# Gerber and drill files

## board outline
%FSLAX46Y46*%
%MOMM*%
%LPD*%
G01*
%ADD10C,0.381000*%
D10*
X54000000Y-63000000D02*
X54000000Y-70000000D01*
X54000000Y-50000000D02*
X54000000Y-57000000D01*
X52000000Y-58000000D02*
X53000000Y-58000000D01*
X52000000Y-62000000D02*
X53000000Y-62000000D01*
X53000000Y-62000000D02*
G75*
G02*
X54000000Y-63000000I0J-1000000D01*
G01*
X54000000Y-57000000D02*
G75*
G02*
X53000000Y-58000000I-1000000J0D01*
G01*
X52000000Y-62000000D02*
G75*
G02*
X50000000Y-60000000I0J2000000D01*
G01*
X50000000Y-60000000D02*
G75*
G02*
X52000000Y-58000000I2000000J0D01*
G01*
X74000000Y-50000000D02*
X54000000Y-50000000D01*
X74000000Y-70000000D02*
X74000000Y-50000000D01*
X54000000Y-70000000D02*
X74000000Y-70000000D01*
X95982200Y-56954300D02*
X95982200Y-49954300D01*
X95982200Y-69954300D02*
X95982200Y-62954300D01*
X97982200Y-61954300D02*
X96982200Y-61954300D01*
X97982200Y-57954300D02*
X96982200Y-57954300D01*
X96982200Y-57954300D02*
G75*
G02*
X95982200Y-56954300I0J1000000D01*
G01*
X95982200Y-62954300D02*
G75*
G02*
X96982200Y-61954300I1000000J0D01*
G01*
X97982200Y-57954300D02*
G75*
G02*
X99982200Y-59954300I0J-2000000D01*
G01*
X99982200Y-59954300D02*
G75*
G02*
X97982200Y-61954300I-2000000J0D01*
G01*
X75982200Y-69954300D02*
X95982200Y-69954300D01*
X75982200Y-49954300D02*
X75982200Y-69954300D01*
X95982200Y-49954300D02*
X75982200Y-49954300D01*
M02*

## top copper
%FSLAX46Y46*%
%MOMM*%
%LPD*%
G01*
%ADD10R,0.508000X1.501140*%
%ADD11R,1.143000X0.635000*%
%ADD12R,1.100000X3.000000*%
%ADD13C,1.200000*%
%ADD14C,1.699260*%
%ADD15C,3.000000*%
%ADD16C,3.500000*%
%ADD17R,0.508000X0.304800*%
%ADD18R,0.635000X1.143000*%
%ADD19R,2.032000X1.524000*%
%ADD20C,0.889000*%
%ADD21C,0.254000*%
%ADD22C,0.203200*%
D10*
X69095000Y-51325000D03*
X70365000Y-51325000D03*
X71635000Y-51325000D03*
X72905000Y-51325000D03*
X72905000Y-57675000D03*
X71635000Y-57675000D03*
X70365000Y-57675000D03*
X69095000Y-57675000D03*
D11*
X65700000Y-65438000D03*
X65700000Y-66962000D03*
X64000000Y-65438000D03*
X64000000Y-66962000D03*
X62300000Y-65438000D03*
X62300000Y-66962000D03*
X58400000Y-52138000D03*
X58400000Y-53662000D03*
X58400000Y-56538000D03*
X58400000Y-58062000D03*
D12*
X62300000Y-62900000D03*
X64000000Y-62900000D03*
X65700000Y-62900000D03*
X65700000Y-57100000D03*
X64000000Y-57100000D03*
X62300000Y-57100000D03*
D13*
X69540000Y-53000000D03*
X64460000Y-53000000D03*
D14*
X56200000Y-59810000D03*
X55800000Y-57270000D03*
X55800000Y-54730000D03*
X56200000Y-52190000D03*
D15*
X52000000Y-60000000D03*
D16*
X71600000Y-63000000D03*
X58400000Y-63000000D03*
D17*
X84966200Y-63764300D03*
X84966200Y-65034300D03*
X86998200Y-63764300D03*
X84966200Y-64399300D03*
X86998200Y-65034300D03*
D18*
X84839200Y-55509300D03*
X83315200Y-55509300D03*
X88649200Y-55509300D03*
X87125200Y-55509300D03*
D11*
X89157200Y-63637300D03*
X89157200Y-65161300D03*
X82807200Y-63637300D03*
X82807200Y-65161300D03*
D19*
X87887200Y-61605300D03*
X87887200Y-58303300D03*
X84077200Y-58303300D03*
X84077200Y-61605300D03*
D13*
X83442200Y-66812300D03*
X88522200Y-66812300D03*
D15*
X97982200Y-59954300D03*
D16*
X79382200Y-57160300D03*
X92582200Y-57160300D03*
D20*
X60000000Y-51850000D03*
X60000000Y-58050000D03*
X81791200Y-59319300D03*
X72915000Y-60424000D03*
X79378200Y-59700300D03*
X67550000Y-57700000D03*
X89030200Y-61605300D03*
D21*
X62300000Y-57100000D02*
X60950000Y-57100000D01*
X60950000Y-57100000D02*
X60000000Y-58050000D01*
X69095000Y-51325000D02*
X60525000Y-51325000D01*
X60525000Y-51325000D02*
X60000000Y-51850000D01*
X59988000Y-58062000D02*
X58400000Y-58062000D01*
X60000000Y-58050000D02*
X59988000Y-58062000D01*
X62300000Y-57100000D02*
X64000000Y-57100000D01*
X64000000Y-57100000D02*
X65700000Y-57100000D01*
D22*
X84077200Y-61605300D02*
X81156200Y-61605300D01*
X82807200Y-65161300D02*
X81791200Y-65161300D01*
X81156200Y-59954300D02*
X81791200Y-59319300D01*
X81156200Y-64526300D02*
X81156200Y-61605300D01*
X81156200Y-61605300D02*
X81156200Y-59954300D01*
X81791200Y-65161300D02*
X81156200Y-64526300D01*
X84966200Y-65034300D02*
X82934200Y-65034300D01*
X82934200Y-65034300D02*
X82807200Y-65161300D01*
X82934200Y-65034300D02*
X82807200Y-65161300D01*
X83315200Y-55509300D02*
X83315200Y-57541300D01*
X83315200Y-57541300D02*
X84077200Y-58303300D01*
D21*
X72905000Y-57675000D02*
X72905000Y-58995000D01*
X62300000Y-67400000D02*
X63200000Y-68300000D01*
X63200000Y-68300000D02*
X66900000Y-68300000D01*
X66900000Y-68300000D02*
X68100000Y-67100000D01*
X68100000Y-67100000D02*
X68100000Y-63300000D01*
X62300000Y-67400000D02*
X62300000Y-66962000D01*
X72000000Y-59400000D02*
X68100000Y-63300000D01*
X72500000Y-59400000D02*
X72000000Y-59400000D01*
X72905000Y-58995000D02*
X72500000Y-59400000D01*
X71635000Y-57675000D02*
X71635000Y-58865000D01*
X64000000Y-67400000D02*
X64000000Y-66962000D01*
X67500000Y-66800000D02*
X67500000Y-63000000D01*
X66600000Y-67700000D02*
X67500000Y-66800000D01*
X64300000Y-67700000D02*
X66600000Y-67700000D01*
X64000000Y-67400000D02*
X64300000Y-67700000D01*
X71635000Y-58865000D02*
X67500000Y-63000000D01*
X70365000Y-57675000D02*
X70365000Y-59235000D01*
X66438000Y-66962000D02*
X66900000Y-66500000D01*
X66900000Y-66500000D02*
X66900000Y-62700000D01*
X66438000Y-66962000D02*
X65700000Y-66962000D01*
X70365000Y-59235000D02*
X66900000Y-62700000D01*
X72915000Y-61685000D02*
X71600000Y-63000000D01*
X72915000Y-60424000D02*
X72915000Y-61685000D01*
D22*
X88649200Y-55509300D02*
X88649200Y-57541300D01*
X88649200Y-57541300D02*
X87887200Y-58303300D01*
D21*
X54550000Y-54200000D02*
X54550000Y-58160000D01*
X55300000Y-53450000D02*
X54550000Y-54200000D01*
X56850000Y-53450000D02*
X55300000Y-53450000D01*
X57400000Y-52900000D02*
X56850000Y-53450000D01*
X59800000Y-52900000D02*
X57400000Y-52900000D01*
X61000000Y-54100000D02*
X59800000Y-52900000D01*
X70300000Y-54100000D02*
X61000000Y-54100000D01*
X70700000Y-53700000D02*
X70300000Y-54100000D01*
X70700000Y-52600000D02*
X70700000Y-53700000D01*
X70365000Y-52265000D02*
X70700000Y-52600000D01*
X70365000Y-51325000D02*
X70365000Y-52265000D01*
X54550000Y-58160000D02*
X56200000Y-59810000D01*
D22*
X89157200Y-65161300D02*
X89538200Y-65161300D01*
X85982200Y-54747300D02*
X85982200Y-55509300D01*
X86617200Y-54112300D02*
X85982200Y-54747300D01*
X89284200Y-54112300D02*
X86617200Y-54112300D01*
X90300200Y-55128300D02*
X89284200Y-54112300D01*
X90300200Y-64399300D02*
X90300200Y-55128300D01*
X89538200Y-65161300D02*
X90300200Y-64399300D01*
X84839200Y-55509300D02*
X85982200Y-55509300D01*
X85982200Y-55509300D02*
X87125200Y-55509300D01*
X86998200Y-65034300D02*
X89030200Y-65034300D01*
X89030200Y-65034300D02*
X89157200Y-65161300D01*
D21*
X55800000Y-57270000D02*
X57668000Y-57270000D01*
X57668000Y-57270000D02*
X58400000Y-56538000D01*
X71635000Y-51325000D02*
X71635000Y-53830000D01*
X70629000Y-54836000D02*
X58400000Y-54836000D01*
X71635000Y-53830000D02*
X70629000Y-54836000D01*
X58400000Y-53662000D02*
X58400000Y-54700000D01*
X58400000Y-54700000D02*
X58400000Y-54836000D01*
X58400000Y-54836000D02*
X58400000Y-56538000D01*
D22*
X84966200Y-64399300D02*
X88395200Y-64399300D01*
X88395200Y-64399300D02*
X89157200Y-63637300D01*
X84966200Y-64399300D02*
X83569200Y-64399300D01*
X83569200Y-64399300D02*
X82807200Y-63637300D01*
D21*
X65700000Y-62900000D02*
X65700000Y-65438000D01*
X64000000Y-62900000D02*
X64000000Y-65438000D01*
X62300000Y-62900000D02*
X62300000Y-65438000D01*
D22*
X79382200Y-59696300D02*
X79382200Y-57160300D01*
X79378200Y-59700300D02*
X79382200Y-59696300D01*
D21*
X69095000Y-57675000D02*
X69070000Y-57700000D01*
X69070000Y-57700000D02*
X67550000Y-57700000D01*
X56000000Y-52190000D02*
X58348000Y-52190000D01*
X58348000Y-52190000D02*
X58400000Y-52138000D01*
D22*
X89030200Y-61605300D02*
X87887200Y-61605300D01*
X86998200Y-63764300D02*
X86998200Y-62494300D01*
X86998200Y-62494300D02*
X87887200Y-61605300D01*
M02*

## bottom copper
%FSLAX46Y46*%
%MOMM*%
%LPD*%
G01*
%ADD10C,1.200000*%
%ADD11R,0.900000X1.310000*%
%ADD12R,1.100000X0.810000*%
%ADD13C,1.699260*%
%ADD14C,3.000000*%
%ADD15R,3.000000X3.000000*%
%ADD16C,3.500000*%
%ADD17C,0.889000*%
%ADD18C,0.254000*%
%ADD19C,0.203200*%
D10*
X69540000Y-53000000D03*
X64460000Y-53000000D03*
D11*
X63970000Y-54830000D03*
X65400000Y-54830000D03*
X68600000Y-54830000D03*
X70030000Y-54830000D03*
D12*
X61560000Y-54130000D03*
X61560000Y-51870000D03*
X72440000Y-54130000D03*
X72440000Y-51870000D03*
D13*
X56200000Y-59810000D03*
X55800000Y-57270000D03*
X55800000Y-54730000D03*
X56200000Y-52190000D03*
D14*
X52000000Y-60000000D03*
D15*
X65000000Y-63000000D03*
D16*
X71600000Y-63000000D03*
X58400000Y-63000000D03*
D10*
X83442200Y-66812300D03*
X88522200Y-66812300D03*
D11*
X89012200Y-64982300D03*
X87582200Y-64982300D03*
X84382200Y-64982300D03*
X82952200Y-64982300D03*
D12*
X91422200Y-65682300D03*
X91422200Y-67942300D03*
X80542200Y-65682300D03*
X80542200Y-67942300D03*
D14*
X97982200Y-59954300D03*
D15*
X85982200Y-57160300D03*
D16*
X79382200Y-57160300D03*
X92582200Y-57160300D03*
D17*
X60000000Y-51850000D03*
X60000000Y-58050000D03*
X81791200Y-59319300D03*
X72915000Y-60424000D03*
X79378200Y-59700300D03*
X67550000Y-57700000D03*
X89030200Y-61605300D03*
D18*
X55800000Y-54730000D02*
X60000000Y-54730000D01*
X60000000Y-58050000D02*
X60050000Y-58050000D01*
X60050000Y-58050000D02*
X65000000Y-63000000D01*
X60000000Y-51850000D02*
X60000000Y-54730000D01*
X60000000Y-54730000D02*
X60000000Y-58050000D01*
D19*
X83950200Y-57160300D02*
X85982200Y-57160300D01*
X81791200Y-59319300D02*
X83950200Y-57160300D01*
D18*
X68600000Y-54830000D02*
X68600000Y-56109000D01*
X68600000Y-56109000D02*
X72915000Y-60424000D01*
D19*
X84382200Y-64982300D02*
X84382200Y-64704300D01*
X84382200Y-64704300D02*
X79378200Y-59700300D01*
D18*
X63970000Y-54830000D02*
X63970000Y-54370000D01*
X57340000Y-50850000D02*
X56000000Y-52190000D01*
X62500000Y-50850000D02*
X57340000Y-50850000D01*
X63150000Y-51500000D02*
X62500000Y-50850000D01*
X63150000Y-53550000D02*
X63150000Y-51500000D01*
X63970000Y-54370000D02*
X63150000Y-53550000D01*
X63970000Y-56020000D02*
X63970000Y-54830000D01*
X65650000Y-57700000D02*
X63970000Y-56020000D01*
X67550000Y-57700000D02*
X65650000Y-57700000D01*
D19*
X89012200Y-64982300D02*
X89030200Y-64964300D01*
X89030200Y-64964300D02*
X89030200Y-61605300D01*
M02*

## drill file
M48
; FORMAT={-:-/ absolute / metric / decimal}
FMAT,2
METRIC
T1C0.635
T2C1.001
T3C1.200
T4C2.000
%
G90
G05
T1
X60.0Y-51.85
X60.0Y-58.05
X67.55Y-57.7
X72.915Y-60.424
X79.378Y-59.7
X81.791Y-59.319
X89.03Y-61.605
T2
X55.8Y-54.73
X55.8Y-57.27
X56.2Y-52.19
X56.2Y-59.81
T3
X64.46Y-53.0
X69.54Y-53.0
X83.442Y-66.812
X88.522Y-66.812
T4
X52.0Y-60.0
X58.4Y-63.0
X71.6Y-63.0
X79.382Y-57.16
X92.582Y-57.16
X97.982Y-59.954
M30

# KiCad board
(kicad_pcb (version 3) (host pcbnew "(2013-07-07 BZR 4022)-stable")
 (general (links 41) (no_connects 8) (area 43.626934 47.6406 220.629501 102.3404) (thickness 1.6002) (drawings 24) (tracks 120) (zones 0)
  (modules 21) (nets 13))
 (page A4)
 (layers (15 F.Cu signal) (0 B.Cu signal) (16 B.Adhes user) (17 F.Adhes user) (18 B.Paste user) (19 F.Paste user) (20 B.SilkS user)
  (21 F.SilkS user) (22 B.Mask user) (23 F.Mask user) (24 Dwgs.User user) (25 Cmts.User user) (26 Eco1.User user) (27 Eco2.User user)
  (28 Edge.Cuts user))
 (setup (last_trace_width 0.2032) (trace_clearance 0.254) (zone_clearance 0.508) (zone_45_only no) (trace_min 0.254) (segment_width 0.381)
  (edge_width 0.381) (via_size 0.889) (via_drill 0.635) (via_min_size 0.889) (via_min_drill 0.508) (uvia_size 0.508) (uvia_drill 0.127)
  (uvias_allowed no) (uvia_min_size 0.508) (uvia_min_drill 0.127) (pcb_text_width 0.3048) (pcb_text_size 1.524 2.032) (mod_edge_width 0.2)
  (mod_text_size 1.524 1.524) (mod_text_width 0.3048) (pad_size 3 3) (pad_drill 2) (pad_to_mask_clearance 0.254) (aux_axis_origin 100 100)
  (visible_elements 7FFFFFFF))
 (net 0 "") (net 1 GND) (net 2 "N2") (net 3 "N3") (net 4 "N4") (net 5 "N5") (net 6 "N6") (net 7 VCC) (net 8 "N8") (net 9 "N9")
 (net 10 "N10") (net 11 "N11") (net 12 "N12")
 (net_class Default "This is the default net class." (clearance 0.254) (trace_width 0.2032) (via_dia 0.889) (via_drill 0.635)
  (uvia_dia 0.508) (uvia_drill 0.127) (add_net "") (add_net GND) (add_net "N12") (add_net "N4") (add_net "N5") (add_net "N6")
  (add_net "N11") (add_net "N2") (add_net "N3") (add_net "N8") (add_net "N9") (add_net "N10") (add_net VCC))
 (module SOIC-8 (layer F.Cu) (at 71 54.5)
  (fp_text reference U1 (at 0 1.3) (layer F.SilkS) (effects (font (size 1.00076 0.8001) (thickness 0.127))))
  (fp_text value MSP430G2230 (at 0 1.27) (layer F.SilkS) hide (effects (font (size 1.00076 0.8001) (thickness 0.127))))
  (pad 8 smd rect (at -1.905 -3.175) (size 0.508 1.50114) (layers F.Cu F.Paste F.Mask) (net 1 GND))
  (pad 7 smd rect (at -0.635 -3.175) (size 0.508 1.50114) (layers F.Cu F.Paste F.Mask) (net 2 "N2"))
  (pad 6 smd rect (at 0.635 -3.175) (size 0.508 1.50114) (layers F.Cu F.Paste F.Mask) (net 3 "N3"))
  (pad 5 smd rect (at 1.905 -3.175) (size 0.508 1.50114) (layers F.Cu F.Paste F.Mask))
  (pad 4 smd rect (at 1.905 3.175) (size 0.508 1.50114) (layers F.Cu F.Paste F.Mask) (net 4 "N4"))
  (pad 3 smd rect (at 0.635 3.175) (size 0.508 1.50114) (layers F.Cu F.Paste F.Mask) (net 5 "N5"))
  (pad 2 smd rect (at -0.635 3.175) (size 0.508 1.50114) (layers F.Cu F.Paste F.Mask) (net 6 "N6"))
  (pad 1 smd rect (at -1.905 3.175) (size 0.508 1.50114) (layers F.Cu F.Paste F.Mask) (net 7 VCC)))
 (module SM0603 (layer F.Cu) (at 65.7 66.2 270)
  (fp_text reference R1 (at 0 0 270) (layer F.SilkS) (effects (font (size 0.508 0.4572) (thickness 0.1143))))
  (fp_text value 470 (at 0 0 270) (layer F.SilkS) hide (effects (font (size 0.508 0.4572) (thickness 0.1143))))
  (pad 1 smd rect (at -0.762 0 270) (size 0.635 1.143) (layers F.Cu F.Paste F.Mask) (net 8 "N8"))
  (pad 2 smd rect (at 0.762 0 270) (size 0.635 1.143) (layers F.Cu F.Paste F.Mask) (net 6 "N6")))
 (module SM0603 (layer F.Cu) (at 64 66.2 270)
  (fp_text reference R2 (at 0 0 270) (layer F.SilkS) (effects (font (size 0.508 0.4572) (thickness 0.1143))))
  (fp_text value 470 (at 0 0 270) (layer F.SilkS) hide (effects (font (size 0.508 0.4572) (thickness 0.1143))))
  (pad 1 smd rect (at -0.762 0 270) (size 0.635 1.143) (layers F.Cu F.Paste F.Mask) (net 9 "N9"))
  (pad 2 smd rect (at 0.762 0 270) (size 0.635 1.143) (layers F.Cu F.Paste F.Mask) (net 5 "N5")))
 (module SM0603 (layer F.Cu) (at 62.3 66.2 270)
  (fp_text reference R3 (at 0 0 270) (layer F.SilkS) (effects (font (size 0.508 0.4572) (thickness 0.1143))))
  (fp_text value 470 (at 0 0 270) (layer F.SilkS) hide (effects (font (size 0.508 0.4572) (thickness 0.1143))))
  (pad 1 smd rect (at -0.762 0 270) (size 0.635 1.143) (layers F.Cu F.Paste F.Mask) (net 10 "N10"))
  (pad 2 smd rect (at 0.762 0 270) (size 0.635 1.143) (layers F.Cu F.Paste F.Mask) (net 4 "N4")))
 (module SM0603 (layer F.Cu) (at 58.4 52.9 270)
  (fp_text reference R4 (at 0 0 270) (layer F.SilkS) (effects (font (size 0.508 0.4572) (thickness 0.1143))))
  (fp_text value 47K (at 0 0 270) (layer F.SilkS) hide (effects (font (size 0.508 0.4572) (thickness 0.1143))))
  (pad 1 smd rect (at -0.762 0 270) (size 0.635 1.143) (layers F.Cu F.Paste F.Mask) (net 7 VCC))
  (pad 2 smd rect (at 0.762 0 270) (size 0.635 1.143) (layers F.Cu F.Paste F.Mask) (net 3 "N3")))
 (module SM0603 (layer F.Cu) (at 58.4 57.3 270)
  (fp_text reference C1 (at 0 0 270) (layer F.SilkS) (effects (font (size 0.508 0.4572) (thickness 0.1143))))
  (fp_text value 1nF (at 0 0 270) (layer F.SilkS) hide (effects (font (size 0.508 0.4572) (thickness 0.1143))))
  (pad 1 smd rect (at -0.762 0 270) (size 0.635 1.143) (layers F.Cu F.Paste F.Mask) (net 3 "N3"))
  (pad 2 smd rect (at 0.762 0 270) (size 0.635 1.143) (layers F.Cu F.Paste F.Mask) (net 1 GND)))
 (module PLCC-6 (layer F.Cu) (at 64 60)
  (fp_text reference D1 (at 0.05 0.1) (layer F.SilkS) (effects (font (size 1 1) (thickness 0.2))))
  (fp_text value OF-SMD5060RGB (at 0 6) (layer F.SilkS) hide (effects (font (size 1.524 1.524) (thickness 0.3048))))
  (pad 1 smd rect (at -1.7 2.9) (size 1.1 3) (layers F.Cu F.Paste F.Mask) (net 10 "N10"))
  (pad 2 smd rect (at 0 2.9) (size 1.1 3) (layers F.Cu F.Paste F.Mask) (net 9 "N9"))
  (pad 3 smd rect (at 1.7 2.9) (size 1.1 3) (layers F.Cu F.Paste F.Mask) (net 8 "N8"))
  (pad 4 smd rect (at 1.7 -2.9) (size 1.1 3) (layers F.Cu F.Paste F.Mask) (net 1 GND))
  (pad 5 smd rect (at 0 -2.9) (size 1.1 3) (layers F.Cu F.Paste F.Mask) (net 1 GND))
  (pad 6 smd rect (at -1.7 -2.9) (size 1.1 3) (layers F.Cu F.Paste F.Mask) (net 1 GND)))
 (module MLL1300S (layer B.Cu) (at 67 53)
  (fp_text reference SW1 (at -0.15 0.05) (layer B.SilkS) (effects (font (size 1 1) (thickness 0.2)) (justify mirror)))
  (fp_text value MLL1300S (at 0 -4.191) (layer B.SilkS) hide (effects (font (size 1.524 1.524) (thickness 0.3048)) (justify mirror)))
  (pad ~ thru_hole circle (at 2.54 0) (size 1.2 1.2) (drill 1.2) (layers *.Cu *.Mask B.SilkS))
  (pad ~ thru_hole circle (at -2.54 0) (size 1.2 1.2) (drill 1.2) (layers *.Cu *.Mask B.SilkS))
  (pad 1 smd rect (at -3.03 1.83) (size 0.9 1.31) (layers B.Cu B.Paste B.Mask) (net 7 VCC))
  (pad 2 smd rect (at -1.6 1.83) (size 0.9 1.31) (layers B.Cu B.Paste B.Mask))
  (pad 3 smd rect (at 1.6 1.83) (size 0.9 1.31) (layers B.Cu B.Paste B.Mask) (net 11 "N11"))
  (pad 4 smd rect (at 3.03 1.83) (size 0.9 1.31) (layers B.Cu B.Paste B.Mask))
  (pad ~ smd rect (at -5.44 1.13) (size 1.1 0.81) (layers B.Cu B.Paste B.Mask))
  (pad ~ smd rect (at -5.44 -1.13) (size 1.1 0.81) (layers B.Cu B.Paste B.Mask))
  (pad ~ smd rect (at 5.44 1.13) (size 1.1 0.81) (layers B.Cu B.Paste B.Mask))
  (pad ~ smd rect (at 5.44 -1.13) (size 1.1 0.81) (layers B.Cu B.Paste B.Mask)))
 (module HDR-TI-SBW (layer F.Cu) (at 56 56 90)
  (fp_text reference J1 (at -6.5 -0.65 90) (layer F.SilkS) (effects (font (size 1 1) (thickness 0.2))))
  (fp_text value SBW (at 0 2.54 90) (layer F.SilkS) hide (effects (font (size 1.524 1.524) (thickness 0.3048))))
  (pad 1 thru_hole circle (at -3.81 0.2 90) (size 1.69926 1.69926) (drill 1.00076) (layers *.Cu *.Mask F.SilkS) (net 2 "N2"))
  (pad 2 thru_hole circle (at -1.27 -0.2 90) (size 1.69926 1.69926) (drill 1.00076) (layers *.Cu *.Mask F.SilkS) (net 3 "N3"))
  (pad 3 thru_hole circle (at 1.27 -0.2 90) (size 1.69926 1.69926) (drill 1.00076) (layers *.Cu *.Mask F.SilkS) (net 1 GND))
  (pad 4 thru_hole circle (at 3.81 0.2 90) (size 1.69926 1.69926) (drill 1.00076) (layers *.Cu *.Mask F.SilkS) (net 7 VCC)))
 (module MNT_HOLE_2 (layer F.Cu) (at 52 60)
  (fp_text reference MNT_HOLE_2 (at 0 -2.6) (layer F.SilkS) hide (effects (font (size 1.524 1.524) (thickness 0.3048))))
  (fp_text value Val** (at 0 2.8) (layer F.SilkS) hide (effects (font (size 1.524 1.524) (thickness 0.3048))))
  (pad "" thru_hole circle (at 0 0) (size 3 3) (drill 2) (layers *.Cu *.Mask F.SilkS)))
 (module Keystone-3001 (layer B.Cu) (at 65 63)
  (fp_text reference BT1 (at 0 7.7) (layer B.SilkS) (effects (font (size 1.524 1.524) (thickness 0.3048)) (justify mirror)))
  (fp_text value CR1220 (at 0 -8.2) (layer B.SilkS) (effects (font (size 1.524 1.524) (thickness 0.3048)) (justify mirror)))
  (pad 2 smd rect (at 0 0) (size 3 3) (layers B.Cu B.Paste B.Mask) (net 1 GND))
  (pad 1 thru_hole circle (at 6.6 0) (size 3.5 3.5) (drill 2) (layers F.Cu F.Mask) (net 11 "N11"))
  (pad 1 thru_hole circle (at -6.6 0) (size 3.5 3.5) (drill 2) (layers F.Cu F.Mask) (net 11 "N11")))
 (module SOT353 (layer F.Cu) (at 85.9822 64.3993)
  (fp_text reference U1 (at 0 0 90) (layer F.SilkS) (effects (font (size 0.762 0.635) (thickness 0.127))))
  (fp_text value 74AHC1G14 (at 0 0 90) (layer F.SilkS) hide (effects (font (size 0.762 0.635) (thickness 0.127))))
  (pad 1 smd rect (at -1.016 -0.635) (size 0.508 0.3048) (layers F.Cu F.Paste F.Mask))
  (pad 3 smd rect (at -1.016 0.635) (size 0.508 0.3048) (layers F.Cu F.Paste F.Mask) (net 1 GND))
  (pad 5 smd rect (at 1.016 -0.635) (size 0.508 0.3048) (layers F.Cu F.Paste F.Mask) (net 7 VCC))
  (pad 2 smd rect (at -1.016 0) (size 0.508 0.3048) (layers F.Cu F.Paste F.Mask) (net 3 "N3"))
  (pad 4 smd rect (at 1.016 0.635) (size 0.508 0.3048) (layers F.Cu F.Paste F.Mask) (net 2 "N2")))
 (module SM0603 (layer F.Cu) (at 84.0772 55.5093 180)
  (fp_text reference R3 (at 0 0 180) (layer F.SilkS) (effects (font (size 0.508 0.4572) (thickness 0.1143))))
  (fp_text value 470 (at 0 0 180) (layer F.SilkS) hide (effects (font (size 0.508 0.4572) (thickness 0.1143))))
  (pad 1 smd rect (at -0.762 0 180) (size 0.635 1.143) (layers F.Cu F.Paste F.Mask) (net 2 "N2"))
  (pad 2 smd rect (at 0.762 0 180) (size 0.635 1.143) (layers F.Cu F.Paste F.Mask) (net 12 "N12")))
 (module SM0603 (layer F.Cu) (at 87.8872 55.5093 180)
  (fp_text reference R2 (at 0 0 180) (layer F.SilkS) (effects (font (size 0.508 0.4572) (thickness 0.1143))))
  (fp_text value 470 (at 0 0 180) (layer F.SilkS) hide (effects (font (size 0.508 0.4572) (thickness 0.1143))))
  (pad 1 smd rect (at -0.762 0 180) (size 0.635 1.143) (layers F.Cu F.Paste F.Mask) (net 11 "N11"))
  (pad 2 smd rect (at 0.762 0 180) (size 0.635 1.143) (layers F.Cu F.Paste F.Mask) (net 2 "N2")))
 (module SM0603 (layer F.Cu) (at 89.1572 64.3993 270)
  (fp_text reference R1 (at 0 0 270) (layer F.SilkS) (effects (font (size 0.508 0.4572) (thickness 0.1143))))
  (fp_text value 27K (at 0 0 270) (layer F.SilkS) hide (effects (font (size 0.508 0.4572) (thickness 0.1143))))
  (pad 1 smd rect (at -0.762 0 270) (size 0.635 1.143) (layers F.Cu F.Paste F.Mask) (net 3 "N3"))
  (pad 2 smd rect (at 0.762 0 270) (size 0.635 1.143) (layers F.Cu F.Paste F.Mask) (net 2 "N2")))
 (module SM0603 (layer F.Cu) (at 82.8072 64.3993 270)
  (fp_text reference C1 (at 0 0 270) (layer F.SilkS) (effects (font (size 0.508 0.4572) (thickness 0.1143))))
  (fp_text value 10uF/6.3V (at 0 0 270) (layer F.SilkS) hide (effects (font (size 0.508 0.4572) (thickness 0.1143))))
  (pad 1 smd rect (at -0.762 0 270) (size 0.635 1.143) (layers F.Cu F.Paste F.Mask) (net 3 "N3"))
  (pad 2 smd rect (at 0.762 0 270) (size 0.635 1.143) (layers F.Cu F.Paste F.Mask) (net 1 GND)))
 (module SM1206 (layer F.Cu) (at 87.8872 59.9543 90)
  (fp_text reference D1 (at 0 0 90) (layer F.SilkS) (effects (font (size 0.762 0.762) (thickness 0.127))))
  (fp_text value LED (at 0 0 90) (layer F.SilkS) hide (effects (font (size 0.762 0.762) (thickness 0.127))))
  (pad 1 smd rect (at -1.651 0 90) (size 1.524 2.032) (layers F.Cu F.Paste F.Mask) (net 7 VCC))
  (pad 2 smd rect (at 1.651 0 90) (size 1.524 2.032) (layers F.Cu F.Paste F.Mask) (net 11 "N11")))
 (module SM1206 (layer F.Cu) (at 84.0772 59.9543 270)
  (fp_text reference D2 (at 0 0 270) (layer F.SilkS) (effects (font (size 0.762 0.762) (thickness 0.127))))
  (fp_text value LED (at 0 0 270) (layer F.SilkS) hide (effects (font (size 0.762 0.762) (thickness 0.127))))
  (pad 1 smd rect (at -1.651 0 270) (size 1.524 2.032) (layers F.Cu F.Paste F.Mask) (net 12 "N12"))
  (pad 2 smd rect (at 1.651 0 270) (size 1.524 2.032) (layers F.Cu F.Paste F.Mask) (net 1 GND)))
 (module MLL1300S (layer B.Cu) (at 85.9822 66.8123 180)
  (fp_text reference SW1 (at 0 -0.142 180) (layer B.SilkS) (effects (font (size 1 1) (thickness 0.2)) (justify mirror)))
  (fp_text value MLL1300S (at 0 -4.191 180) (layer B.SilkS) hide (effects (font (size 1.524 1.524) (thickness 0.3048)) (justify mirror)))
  (pad ~ thru_hole circle (at 2.54 0 180) (size 1.2 1.2) (drill 1.2) (layers *.Cu *.Mask B.SilkS))
  (pad ~ thru_hole circle (at -2.54 0 180) (size 1.2 1.2) (drill 1.2) (layers *.Cu *.Mask B.SilkS))
  (pad 1 smd rect (at -3.03 1.83 180) (size 0.9 1.31) (layers B.Cu B.Paste B.Mask) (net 7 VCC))
  (pad 2 smd rect (at -1.6 1.83 180) (size 0.9 1.31) (layers B.Cu B.Paste B.Mask))
  (pad 3 smd rect (at 1.6 1.83 180) (size 0.9 1.31) (layers B.Cu B.Paste B.Mask) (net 10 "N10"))
  (pad 4 smd rect (at 3.03 1.83 180) (size 0.9 1.31) (layers B.Cu B.Paste B.Mask))
  (pad ~ smd rect (at -5.44 1.13 180) (size 1.1 0.81) (layers B.Cu B.Paste B.Mask))
  (pad ~ smd rect (at -5.44 -1.13 180) (size 1.1 0.81) (layers B.Cu B.Paste B.Mask))
  (pad ~ smd rect (at 5.44 1.13 180) (size 1.1 0.81) (layers B.Cu B.Paste B.Mask))
  (pad ~ smd rect (at 5.44 -1.13 180) (size 1.1 0.81) (layers B.Cu B.Paste B.Mask)))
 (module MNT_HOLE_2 (layer F.Cu) (at 97.9822 59.9543 180)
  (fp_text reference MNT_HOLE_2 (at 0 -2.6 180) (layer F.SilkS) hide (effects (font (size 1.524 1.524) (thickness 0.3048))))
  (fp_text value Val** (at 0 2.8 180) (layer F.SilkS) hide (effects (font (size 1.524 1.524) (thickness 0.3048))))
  (pad "" thru_hole circle (at 0 0 180) (size 3 3) (drill 2) (layers *.Cu *.Mask F.SilkS)))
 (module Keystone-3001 (layer B.Cu) (at 85.9822 57.1603 180)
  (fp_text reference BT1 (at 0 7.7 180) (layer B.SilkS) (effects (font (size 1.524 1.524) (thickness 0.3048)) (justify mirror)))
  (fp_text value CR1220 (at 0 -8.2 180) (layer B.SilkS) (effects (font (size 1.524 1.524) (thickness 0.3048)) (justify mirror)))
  (pad 2 smd rect (at 0 0 180) (size 3 3) (layers B.Cu B.Paste B.Mask) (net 1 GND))
  (pad 1 thru_hole circle (at 6.6 0 180) (size 3.5 3.5) (drill 2) (layers F.Cu F.Mask) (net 10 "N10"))
  (pad 1 thru_hole circle (at -6.6 0 180) (size 3.5 3.5) (drill 2) (layers F.Cu F.Mask) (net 10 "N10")))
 (gr_line (start 54 63) (end 54 70) (angle 90) (layer Edge.Cuts) (width 0.381))
 (gr_line (start 54 50) (end 54 57) (angle 90) (layer Edge.Cuts) (width 0.381))
 (gr_line (start 52 58) (end 53 58) (angle 90) (layer Edge.Cuts) (width 0.381))
 (gr_line (start 52 62) (end 53 62) (angle 90) (layer Edge.Cuts) (width 0.381))
 (gr_arc (start 53 63) (end 53 62) (angle 90) (layer Edge.Cuts) (width 0.381))
 (gr_arc (start 53 57) (end 54 57) (angle 90) (layer Edge.Cuts) (width 0.381))
 (gr_arc (start 52 60) (end 52 62) (angle 90) (layer Edge.Cuts) (width 0.381))
 (gr_arc (start 52 60) (end 50 60) (angle 90) (layer Edge.Cuts) (width 0.381))
 (gr_line (start 74 50) (end 54 50) (angle 90) (layer Edge.Cuts) (width 0.381))
 (gr_line (start 74 70) (end 74 50) (angle 90) (layer Edge.Cuts) (width 0.381))
 (gr_line (start 54 70) (end 74 70) (angle 90) (layer Edge.Cuts) (width 0.381))
 (gr_line (start 95.9822 56.9543) (end 95.9822 49.9543) (angle 90) (layer Edge.Cuts) (width 0.381))
 (gr_line (start 95.9822 69.9543) (end 95.9822 62.9543) (angle 90) (layer Edge.Cuts) (width 0.381))
 (gr_line (start 97.9822 61.9543) (end 96.9822 61.9543) (angle 90) (layer Edge.Cuts) (width 0.381))
 (gr_line (start 97.9822 57.9543) (end 96.9822 57.9543) (angle 90) (layer Edge.Cuts) (width 0.381))
 (gr_arc (start 96.9822 56.9543) (end 96.9822 57.9543) (angle 90) (layer Edge.Cuts) (width 0.381))
 (gr_arc (start 96.9822 62.9543) (end 95.9822 62.9543) (angle 90) (layer Edge.Cuts) (width 0.381))
 (gr_arc (start 97.9822 59.9543) (end 97.9822 57.9543) (angle 90) (layer Edge.Cuts) (width 0.381))
 (gr_arc (start 97.9822 59.9543) (end 99.9822 59.9543) (angle 90) (layer Edge.Cuts) (width 0.381))
 (gr_line (start 75.9822 69.9543) (end 95.9822 69.9543) (angle 90) (layer Edge.Cuts) (width 0.381))
 (gr_line (start 75.9822 49.9543) (end 75.9822 69.9543) (angle 90) (layer Edge.Cuts) (width 0.381))
 (gr_line (start 95.9822 49.9543) (end 75.9822 49.9543) (angle 90) (layer Edge.Cuts) (width 0.381))
 (segment (start 55.8 54.73) (end 60 54.73) (width 0.254) (layer B.Cu) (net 1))
 (segment (start 60 58.05) (end 60.05 58.05) (width 0.254) (layer B.Cu) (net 1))
 (segment (start 60.05 58.05) (end 65 63) (width 0.254) (layer B.Cu) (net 1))
 (segment (start 62.3 57.1) (end 60.95 57.1) (width 0.254) (layer F.Cu) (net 1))
 (segment (start 60.95 57.1) (end 60 58.05) (width 0.254) (layer F.Cu) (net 1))
 (segment (start 69.095 51.325) (end 60.525 51.325) (width 0.254) (layer F.Cu) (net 1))
 (segment (start 60.525 51.325) (end 60 51.85) (width 0.254) (layer F.Cu) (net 1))
 (via (at 60 51.85) (size 0.889) (layers F.Cu B.Cu) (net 1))
 (segment (start 60 51.85) (end 60 54.73) (width 0.254) (layer B.Cu) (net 1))
 (segment (start 60 54.73) (end 60 58.05) (width 0.254) (layer B.Cu) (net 1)) (via (at 60 58.05) (size 0.889) (layers F.Cu B.Cu) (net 1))
 (segment (start 59.988 58.062) (end 58.4 58.062) (width 0.254) (layer F.Cu) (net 1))
 (segment (start 60 58.05) (end 59.988 58.062) (width 0.254) (layer F.Cu) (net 1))
 (segment (start 62.3 57.1) (end 64 57.1) (width 0.254) (layer F.Cu) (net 1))
 (segment (start 64 57.1) (end 65.7 57.1) (width 0.254) (layer F.Cu) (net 1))
 (segment (start 84.0772 61.6053) (end 81.1562 61.6053) (width 0.2032) (layer F.Cu) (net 1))
 (segment (start 82.8072 65.1613) (end 81.7912 65.1613) (width 0.2032) (layer F.Cu) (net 1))
 (segment (start 83.9502 57.1603) (end 85.9822 57.1603) (width 0.2032) (layer B.Cu) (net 1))
 (segment (start 81.7912 59.3193) (end 83.9502 57.1603) (width 0.2032) (layer B.Cu) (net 1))
 (via (at 81.7912 59.3193) (size 0.889) (layers F.Cu B.Cu) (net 1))
 (segment (start 81.1562 59.9543) (end 81.7912 59.3193) (width 0.2032) (layer F.Cu) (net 1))
 (segment (start 81.1562 64.5263) (end 81.1562 61.6053) (width 0.2032) (layer F.Cu) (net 1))
 (segment (start 81.1562 61.6053) (end 81.1562 59.9543) (width 0.2032) (layer F.Cu) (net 1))
 (segment (start 81.7912 65.1613) (end 81.1562 64.5263) (width 0.2032) (layer F.Cu) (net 1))
 (segment (start 84.9662 65.0343) (end 82.9342 65.0343) (width 0.2032) (layer F.Cu) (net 1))
 (segment (start 82.9342 65.0343) (end 82.8072 65.1613) (width 0.2032) (layer F.Cu) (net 1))
 (segment (start 82.9342 65.0343) (end 82.8072 65.1613) (width 0.2032) (layer F.Cu) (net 1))
 (segment (start 83.3152 55.5093) (end 83.3152 57.5413) (width 0.2032) (layer F.Cu) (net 12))
 (segment (start 83.3152 57.5413) (end 84.0772 58.3033) (width 0.2032) (layer F.Cu) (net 12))
 (segment (start 72.905 57.675) (end 72.905 58.995) (width 0.254) (layer F.Cu) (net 4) (status 10))
 (segment (start 62.3 67.4) (end 63.2 68.3) (width 0.254) (layer F.Cu) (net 4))
 (segment (start 63.2 68.3) (end 66.9 68.3) (width 0.254) (layer F.Cu) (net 4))
 (segment (start 66.9 68.3) (end 68.1 67.1) (width 0.254) (layer F.Cu) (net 4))
 (segment (start 68.1 67.1) (end 68.1 63.3) (width 0.254) (layer F.Cu) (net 4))
 (segment (start 62.3 67.4) (end 62.3 66.962) (width 0.254) (layer F.Cu) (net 4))
 (segment (start 72 59.4) (end 68.1 63.3) (width 0.254) (layer F.Cu) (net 4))
 (segment (start 72.5 59.4) (end 72 59.4) (width 0.254) (layer F.Cu) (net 4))
 (segment (start 72.905 58.995) (end 72.5 59.4) (width 0.254) (layer F.Cu) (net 4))
 (segment (start 71.635 57.675) (end 71.635 58.865) (width 0.254) (layer F.Cu) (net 5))
 (segment (start 64 67.4) (end 64 66.962) (width 0.254) (layer F.Cu) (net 5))
 (segment (start 67.5 66.8) (end 67.5 63) (width 0.254) (layer F.Cu) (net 5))
 (segment (start 66.6 67.7) (end 67.5 66.8) (width 0.254) (layer F.Cu) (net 5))
 (segment (start 64.3 67.7) (end 66.6 67.7) (width 0.254) (layer F.Cu) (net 5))
 (segment (start 64 67.4) (end 64.3 67.7) (width 0.254) (layer F.Cu) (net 5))
 (segment (start 71.635 58.865) (end 67.5 63) (width 0.254) (layer F.Cu) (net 5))
 (segment (start 70.365 57.675) (end 70.365 59.235) (width 0.254) (layer F.Cu) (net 6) (status 10))
 (segment (start 66.438 66.962) (end 66.9 66.5) (width 0.254) (layer F.Cu) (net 6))
 (segment (start 66.9 66.5) (end 66.9 62.7) (width 0.254) (layer F.Cu) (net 6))
 (segment (start 66.438 66.962) (end 65.7 66.962) (width 0.254) (layer F.Cu) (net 6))
 (segment (start 70.365 59.235) (end 66.9 62.7) (width 0.254) (layer F.Cu) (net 6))
 (segment (start 68.6 54.83) (end 68.6 56.109) (width 0.254) (layer B.Cu) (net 11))
 (segment (start 72.915 61.685) (end 71.6 63) (width 0.254) (layer F.Cu) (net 11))
 (segment (start 72.915 60.424) (end 72.915 61.685) (width 0.254) (layer F.Cu) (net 11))
 (via (at 72.915 60.424) (size 0.889) (layers F.Cu B.Cu) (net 11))
 (segment (start 68.6 56.109) (end 72.915 60.424) (width 0.254) (layer B.Cu) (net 11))
 (segment (start 88.6492 55.5093) (end 88.6492 57.5413) (width 0.2032) (layer F.Cu) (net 11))
 (segment (start 88.6492 57.5413) (end 87.8872 58.3033) (width 0.2032) (layer F.Cu) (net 11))
 (segment (start 54.55 54.2) (end 54.55 58.16) (width 0.254) (layer F.Cu) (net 2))
 (segment (start 55.3 53.45) (end 54.55 54.2) (width 0.254) (layer F.Cu) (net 2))
 (segment (start 56.85 53.45) (end 55.3 53.45) (width 0.254) (layer F.Cu) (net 2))
 (segment (start 57.4 52.9) (end 56.85 53.45) (width 0.254) (layer F.Cu) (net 2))
 (segment (start 59.8 52.9) (end 57.4 52.9) (width 0.254) (layer F.Cu) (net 2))
 (segment (start 61 54.1) (end 59.8 52.9) (width 0.254) (layer F.Cu) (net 2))
 (segment (start 70.3 54.1) (end 61 54.1) (width 0.254) (layer F.Cu) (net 2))
 (segment (start 70.7 53.7) (end 70.3 54.1) (width 0.254) (layer F.Cu) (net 2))
 (segment (start 70.7 52.6) (end 70.7 53.7) (width 0.254) (layer F.Cu) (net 2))
 (segment (start 70.365 52.265) (end 70.7 52.6) (width 0.254) (layer F.Cu) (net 2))
 (segment (start 70.365 51.325) (end 70.365 52.265) (width 0.254) (layer F.Cu) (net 2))
 (segment (start 54.55 58.16) (end 56.2 59.81) (width 0.254) (layer F.Cu) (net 2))
 (segment (start 89.1572 65.1613) (end 89.5382 65.1613) (width 0.2032) (layer F.Cu) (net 2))
 (segment (start 85.9822 54.7473) (end 85.9822 55.5093) (width 0.2032) (layer F.Cu) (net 2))
 (segment (start 86.6172 54.1123) (end 85.9822 54.7473) (width 0.2032) (layer F.Cu) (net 2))
 (segment (start 89.2842 54.1123) (end 86.6172 54.1123) (width 0.2032) (layer F.Cu) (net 2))
 (segment (start 90.3002 55.1283) (end 89.2842 54.1123) (width 0.2032) (layer F.Cu) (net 2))
 (segment (start 90.3002 64.3993) (end 90.3002 55.1283) (width 0.2032) (layer F.Cu) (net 2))
 (segment (start 89.5382 65.1613) (end 90.3002 64.3993) (width 0.2032) (layer F.Cu) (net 2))
 (segment (start 84.8392 55.5093) (end 85.9822 55.5093) (width 0.2032) (layer F.Cu) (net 2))
 (segment (start 85.9822 55.5093) (end 87.1252 55.5093) (width 0.2032) (layer F.Cu) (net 2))
 (segment (start 86.9982 65.0343) (end 89.0302 65.0343) (width 0.2032) (layer F.Cu) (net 2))
 (segment (start 89.0302 65.0343) (end 89.1572 65.1613) (width 0.2032) (layer F.Cu) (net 2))
 (segment (start 55.8 57.27) (end 57.668 57.27) (width 0.254) (layer F.Cu) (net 3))
 (segment (start 57.668 57.27) (end 58.4 56.538) (width 0.254) (layer F.Cu) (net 3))
 (segment (start 71.635 51.325) (end 71.635 53.83) (width 0.254) (layer F.Cu) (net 3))
 (segment (start 70.629 54.836) (end 58.4 54.836) (width 0.254) (layer F.Cu) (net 3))
 (segment (start 71.635 53.83) (end 70.629 54.836) (width 0.254) (layer F.Cu) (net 3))
 (segment (start 58.4 53.662) (end 58.4 54.7) (width 0.254) (layer F.Cu) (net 3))
 (segment (start 58.4 54.7) (end 58.4 54.836) (width 0.254) (layer F.Cu) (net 3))
 (segment (start 58.4 54.836) (end 58.4 56.538) (width 0.254) (layer F.Cu) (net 3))
 (segment (start 84.9662 64.3993) (end 88.3952 64.3993) (width 0.2032) (layer F.Cu) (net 3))
 (segment (start 88.3952 64.3993) (end 89.1572 63.6373) (width 0.2032) (layer F.Cu) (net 3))
 (segment (start 84.9662 64.3993) (end 83.5692 64.3993) (width 0.2032) (layer F.Cu) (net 3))
 (segment (start 83.5692 64.3993) (end 82.8072 63.6373) (width 0.2032) (layer F.Cu) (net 3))
 (segment (start 65.7 62.9) (end 65.7 65.438) (width 0.254) (layer F.Cu) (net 8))
 (segment (start 64 62.9) (end 64 65.438) (width 0.254) (layer F.Cu) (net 9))
 (segment (start 62.3 62.9) (end 62.3 65.438) (width 0.254) (layer F.Cu) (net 10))
 (segment (start 84.3822 64.9823) (end 84.3822 64.7043) (width 0.2032) (layer B.Cu) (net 10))
 (segment (start 79.3822 59.6963) (end 79.3822 57.1603) (width 0.2032) (layer F.Cu) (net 10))
 (segment (start 79.3782 59.7003) (end 79.3822 59.6963) (width 0.2032) (layer F.Cu) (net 10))
 (via (at 79.3782 59.7003) (size 0.889) (layers F.Cu B.Cu) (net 10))
 (segment (start 84.3822 64.7043) (end 79.3782 59.7003) (width 0.2032) (layer B.Cu) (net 10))
 (segment (start 63.97 54.83) (end 63.97 54.37) (width 0.254) (layer B.Cu) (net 7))
 (segment (start 57.34 50.85) (end 56 52.19) (width 0.254) (layer B.Cu) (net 7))
 (segment (start 62.5 50.85) (end 57.34 50.85) (width 0.254) (layer B.Cu) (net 7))
 (segment (start 63.15 51.5) (end 62.5 50.85) (width 0.254) (layer B.Cu) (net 7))
 (segment (start 63.15 53.55) (end 63.15 51.5) (width 0.254) (layer B.Cu) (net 7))
 (segment (start 63.97 54.37) (end 63.15 53.55) (width 0.254) (layer B.Cu) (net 7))
 (segment (start 69.095 57.675) (end 69.07 57.7) (width 0.254) (layer F.Cu) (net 7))
 (segment (start 63.97 56.02) (end 63.97 54.83) (width 0.254) (layer B.Cu) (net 7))
 (segment (start 65.65 57.7) (end 63.97 56.02) (width 0.254) (layer B.Cu) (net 7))
 (segment (start 67.55 57.7) (end 65.65 57.7) (width 0.254) (layer B.Cu) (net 7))
 (via (at 67.55 57.7) (size 0.889) (layers F.Cu B.Cu) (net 7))
 (segment (start 69.07 57.7) (end 67.55 57.7) (width 0.254) (layer F.Cu) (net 7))
 (segment (start 56 52.19) (end 58.348 52.19) (width 0.254) (layer F.Cu) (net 7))
 (segment (start 58.348 52.19) (end 58.4 52.138) (width 0.254) (layer F.Cu) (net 7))
 (segment (start 89.0122 64.9823) (end 89.0302 64.9643) (width 0.2032) (layer B.Cu) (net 7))
 (segment (start 89.0302 61.6053) (end 87.8872 61.6053) (width 0.2032) (layer F.Cu) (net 7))
 (via (at 89.0302 61.6053) (size 0.889) (layers F.Cu B.Cu) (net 7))
 (segment (start 89.0302 64.9643) (end 89.0302 61.6053) (width 0.2032) (layer B.Cu) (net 7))
 (segment (start 86.9982 63.7643) (end 86.9982 62.4943) (width 0.2032) (layer F.Cu) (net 7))
 (segment (start 86.9982 62.4943) (end 87.8872 61.6053) (width 0.2032) (layer F.Cu) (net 7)))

